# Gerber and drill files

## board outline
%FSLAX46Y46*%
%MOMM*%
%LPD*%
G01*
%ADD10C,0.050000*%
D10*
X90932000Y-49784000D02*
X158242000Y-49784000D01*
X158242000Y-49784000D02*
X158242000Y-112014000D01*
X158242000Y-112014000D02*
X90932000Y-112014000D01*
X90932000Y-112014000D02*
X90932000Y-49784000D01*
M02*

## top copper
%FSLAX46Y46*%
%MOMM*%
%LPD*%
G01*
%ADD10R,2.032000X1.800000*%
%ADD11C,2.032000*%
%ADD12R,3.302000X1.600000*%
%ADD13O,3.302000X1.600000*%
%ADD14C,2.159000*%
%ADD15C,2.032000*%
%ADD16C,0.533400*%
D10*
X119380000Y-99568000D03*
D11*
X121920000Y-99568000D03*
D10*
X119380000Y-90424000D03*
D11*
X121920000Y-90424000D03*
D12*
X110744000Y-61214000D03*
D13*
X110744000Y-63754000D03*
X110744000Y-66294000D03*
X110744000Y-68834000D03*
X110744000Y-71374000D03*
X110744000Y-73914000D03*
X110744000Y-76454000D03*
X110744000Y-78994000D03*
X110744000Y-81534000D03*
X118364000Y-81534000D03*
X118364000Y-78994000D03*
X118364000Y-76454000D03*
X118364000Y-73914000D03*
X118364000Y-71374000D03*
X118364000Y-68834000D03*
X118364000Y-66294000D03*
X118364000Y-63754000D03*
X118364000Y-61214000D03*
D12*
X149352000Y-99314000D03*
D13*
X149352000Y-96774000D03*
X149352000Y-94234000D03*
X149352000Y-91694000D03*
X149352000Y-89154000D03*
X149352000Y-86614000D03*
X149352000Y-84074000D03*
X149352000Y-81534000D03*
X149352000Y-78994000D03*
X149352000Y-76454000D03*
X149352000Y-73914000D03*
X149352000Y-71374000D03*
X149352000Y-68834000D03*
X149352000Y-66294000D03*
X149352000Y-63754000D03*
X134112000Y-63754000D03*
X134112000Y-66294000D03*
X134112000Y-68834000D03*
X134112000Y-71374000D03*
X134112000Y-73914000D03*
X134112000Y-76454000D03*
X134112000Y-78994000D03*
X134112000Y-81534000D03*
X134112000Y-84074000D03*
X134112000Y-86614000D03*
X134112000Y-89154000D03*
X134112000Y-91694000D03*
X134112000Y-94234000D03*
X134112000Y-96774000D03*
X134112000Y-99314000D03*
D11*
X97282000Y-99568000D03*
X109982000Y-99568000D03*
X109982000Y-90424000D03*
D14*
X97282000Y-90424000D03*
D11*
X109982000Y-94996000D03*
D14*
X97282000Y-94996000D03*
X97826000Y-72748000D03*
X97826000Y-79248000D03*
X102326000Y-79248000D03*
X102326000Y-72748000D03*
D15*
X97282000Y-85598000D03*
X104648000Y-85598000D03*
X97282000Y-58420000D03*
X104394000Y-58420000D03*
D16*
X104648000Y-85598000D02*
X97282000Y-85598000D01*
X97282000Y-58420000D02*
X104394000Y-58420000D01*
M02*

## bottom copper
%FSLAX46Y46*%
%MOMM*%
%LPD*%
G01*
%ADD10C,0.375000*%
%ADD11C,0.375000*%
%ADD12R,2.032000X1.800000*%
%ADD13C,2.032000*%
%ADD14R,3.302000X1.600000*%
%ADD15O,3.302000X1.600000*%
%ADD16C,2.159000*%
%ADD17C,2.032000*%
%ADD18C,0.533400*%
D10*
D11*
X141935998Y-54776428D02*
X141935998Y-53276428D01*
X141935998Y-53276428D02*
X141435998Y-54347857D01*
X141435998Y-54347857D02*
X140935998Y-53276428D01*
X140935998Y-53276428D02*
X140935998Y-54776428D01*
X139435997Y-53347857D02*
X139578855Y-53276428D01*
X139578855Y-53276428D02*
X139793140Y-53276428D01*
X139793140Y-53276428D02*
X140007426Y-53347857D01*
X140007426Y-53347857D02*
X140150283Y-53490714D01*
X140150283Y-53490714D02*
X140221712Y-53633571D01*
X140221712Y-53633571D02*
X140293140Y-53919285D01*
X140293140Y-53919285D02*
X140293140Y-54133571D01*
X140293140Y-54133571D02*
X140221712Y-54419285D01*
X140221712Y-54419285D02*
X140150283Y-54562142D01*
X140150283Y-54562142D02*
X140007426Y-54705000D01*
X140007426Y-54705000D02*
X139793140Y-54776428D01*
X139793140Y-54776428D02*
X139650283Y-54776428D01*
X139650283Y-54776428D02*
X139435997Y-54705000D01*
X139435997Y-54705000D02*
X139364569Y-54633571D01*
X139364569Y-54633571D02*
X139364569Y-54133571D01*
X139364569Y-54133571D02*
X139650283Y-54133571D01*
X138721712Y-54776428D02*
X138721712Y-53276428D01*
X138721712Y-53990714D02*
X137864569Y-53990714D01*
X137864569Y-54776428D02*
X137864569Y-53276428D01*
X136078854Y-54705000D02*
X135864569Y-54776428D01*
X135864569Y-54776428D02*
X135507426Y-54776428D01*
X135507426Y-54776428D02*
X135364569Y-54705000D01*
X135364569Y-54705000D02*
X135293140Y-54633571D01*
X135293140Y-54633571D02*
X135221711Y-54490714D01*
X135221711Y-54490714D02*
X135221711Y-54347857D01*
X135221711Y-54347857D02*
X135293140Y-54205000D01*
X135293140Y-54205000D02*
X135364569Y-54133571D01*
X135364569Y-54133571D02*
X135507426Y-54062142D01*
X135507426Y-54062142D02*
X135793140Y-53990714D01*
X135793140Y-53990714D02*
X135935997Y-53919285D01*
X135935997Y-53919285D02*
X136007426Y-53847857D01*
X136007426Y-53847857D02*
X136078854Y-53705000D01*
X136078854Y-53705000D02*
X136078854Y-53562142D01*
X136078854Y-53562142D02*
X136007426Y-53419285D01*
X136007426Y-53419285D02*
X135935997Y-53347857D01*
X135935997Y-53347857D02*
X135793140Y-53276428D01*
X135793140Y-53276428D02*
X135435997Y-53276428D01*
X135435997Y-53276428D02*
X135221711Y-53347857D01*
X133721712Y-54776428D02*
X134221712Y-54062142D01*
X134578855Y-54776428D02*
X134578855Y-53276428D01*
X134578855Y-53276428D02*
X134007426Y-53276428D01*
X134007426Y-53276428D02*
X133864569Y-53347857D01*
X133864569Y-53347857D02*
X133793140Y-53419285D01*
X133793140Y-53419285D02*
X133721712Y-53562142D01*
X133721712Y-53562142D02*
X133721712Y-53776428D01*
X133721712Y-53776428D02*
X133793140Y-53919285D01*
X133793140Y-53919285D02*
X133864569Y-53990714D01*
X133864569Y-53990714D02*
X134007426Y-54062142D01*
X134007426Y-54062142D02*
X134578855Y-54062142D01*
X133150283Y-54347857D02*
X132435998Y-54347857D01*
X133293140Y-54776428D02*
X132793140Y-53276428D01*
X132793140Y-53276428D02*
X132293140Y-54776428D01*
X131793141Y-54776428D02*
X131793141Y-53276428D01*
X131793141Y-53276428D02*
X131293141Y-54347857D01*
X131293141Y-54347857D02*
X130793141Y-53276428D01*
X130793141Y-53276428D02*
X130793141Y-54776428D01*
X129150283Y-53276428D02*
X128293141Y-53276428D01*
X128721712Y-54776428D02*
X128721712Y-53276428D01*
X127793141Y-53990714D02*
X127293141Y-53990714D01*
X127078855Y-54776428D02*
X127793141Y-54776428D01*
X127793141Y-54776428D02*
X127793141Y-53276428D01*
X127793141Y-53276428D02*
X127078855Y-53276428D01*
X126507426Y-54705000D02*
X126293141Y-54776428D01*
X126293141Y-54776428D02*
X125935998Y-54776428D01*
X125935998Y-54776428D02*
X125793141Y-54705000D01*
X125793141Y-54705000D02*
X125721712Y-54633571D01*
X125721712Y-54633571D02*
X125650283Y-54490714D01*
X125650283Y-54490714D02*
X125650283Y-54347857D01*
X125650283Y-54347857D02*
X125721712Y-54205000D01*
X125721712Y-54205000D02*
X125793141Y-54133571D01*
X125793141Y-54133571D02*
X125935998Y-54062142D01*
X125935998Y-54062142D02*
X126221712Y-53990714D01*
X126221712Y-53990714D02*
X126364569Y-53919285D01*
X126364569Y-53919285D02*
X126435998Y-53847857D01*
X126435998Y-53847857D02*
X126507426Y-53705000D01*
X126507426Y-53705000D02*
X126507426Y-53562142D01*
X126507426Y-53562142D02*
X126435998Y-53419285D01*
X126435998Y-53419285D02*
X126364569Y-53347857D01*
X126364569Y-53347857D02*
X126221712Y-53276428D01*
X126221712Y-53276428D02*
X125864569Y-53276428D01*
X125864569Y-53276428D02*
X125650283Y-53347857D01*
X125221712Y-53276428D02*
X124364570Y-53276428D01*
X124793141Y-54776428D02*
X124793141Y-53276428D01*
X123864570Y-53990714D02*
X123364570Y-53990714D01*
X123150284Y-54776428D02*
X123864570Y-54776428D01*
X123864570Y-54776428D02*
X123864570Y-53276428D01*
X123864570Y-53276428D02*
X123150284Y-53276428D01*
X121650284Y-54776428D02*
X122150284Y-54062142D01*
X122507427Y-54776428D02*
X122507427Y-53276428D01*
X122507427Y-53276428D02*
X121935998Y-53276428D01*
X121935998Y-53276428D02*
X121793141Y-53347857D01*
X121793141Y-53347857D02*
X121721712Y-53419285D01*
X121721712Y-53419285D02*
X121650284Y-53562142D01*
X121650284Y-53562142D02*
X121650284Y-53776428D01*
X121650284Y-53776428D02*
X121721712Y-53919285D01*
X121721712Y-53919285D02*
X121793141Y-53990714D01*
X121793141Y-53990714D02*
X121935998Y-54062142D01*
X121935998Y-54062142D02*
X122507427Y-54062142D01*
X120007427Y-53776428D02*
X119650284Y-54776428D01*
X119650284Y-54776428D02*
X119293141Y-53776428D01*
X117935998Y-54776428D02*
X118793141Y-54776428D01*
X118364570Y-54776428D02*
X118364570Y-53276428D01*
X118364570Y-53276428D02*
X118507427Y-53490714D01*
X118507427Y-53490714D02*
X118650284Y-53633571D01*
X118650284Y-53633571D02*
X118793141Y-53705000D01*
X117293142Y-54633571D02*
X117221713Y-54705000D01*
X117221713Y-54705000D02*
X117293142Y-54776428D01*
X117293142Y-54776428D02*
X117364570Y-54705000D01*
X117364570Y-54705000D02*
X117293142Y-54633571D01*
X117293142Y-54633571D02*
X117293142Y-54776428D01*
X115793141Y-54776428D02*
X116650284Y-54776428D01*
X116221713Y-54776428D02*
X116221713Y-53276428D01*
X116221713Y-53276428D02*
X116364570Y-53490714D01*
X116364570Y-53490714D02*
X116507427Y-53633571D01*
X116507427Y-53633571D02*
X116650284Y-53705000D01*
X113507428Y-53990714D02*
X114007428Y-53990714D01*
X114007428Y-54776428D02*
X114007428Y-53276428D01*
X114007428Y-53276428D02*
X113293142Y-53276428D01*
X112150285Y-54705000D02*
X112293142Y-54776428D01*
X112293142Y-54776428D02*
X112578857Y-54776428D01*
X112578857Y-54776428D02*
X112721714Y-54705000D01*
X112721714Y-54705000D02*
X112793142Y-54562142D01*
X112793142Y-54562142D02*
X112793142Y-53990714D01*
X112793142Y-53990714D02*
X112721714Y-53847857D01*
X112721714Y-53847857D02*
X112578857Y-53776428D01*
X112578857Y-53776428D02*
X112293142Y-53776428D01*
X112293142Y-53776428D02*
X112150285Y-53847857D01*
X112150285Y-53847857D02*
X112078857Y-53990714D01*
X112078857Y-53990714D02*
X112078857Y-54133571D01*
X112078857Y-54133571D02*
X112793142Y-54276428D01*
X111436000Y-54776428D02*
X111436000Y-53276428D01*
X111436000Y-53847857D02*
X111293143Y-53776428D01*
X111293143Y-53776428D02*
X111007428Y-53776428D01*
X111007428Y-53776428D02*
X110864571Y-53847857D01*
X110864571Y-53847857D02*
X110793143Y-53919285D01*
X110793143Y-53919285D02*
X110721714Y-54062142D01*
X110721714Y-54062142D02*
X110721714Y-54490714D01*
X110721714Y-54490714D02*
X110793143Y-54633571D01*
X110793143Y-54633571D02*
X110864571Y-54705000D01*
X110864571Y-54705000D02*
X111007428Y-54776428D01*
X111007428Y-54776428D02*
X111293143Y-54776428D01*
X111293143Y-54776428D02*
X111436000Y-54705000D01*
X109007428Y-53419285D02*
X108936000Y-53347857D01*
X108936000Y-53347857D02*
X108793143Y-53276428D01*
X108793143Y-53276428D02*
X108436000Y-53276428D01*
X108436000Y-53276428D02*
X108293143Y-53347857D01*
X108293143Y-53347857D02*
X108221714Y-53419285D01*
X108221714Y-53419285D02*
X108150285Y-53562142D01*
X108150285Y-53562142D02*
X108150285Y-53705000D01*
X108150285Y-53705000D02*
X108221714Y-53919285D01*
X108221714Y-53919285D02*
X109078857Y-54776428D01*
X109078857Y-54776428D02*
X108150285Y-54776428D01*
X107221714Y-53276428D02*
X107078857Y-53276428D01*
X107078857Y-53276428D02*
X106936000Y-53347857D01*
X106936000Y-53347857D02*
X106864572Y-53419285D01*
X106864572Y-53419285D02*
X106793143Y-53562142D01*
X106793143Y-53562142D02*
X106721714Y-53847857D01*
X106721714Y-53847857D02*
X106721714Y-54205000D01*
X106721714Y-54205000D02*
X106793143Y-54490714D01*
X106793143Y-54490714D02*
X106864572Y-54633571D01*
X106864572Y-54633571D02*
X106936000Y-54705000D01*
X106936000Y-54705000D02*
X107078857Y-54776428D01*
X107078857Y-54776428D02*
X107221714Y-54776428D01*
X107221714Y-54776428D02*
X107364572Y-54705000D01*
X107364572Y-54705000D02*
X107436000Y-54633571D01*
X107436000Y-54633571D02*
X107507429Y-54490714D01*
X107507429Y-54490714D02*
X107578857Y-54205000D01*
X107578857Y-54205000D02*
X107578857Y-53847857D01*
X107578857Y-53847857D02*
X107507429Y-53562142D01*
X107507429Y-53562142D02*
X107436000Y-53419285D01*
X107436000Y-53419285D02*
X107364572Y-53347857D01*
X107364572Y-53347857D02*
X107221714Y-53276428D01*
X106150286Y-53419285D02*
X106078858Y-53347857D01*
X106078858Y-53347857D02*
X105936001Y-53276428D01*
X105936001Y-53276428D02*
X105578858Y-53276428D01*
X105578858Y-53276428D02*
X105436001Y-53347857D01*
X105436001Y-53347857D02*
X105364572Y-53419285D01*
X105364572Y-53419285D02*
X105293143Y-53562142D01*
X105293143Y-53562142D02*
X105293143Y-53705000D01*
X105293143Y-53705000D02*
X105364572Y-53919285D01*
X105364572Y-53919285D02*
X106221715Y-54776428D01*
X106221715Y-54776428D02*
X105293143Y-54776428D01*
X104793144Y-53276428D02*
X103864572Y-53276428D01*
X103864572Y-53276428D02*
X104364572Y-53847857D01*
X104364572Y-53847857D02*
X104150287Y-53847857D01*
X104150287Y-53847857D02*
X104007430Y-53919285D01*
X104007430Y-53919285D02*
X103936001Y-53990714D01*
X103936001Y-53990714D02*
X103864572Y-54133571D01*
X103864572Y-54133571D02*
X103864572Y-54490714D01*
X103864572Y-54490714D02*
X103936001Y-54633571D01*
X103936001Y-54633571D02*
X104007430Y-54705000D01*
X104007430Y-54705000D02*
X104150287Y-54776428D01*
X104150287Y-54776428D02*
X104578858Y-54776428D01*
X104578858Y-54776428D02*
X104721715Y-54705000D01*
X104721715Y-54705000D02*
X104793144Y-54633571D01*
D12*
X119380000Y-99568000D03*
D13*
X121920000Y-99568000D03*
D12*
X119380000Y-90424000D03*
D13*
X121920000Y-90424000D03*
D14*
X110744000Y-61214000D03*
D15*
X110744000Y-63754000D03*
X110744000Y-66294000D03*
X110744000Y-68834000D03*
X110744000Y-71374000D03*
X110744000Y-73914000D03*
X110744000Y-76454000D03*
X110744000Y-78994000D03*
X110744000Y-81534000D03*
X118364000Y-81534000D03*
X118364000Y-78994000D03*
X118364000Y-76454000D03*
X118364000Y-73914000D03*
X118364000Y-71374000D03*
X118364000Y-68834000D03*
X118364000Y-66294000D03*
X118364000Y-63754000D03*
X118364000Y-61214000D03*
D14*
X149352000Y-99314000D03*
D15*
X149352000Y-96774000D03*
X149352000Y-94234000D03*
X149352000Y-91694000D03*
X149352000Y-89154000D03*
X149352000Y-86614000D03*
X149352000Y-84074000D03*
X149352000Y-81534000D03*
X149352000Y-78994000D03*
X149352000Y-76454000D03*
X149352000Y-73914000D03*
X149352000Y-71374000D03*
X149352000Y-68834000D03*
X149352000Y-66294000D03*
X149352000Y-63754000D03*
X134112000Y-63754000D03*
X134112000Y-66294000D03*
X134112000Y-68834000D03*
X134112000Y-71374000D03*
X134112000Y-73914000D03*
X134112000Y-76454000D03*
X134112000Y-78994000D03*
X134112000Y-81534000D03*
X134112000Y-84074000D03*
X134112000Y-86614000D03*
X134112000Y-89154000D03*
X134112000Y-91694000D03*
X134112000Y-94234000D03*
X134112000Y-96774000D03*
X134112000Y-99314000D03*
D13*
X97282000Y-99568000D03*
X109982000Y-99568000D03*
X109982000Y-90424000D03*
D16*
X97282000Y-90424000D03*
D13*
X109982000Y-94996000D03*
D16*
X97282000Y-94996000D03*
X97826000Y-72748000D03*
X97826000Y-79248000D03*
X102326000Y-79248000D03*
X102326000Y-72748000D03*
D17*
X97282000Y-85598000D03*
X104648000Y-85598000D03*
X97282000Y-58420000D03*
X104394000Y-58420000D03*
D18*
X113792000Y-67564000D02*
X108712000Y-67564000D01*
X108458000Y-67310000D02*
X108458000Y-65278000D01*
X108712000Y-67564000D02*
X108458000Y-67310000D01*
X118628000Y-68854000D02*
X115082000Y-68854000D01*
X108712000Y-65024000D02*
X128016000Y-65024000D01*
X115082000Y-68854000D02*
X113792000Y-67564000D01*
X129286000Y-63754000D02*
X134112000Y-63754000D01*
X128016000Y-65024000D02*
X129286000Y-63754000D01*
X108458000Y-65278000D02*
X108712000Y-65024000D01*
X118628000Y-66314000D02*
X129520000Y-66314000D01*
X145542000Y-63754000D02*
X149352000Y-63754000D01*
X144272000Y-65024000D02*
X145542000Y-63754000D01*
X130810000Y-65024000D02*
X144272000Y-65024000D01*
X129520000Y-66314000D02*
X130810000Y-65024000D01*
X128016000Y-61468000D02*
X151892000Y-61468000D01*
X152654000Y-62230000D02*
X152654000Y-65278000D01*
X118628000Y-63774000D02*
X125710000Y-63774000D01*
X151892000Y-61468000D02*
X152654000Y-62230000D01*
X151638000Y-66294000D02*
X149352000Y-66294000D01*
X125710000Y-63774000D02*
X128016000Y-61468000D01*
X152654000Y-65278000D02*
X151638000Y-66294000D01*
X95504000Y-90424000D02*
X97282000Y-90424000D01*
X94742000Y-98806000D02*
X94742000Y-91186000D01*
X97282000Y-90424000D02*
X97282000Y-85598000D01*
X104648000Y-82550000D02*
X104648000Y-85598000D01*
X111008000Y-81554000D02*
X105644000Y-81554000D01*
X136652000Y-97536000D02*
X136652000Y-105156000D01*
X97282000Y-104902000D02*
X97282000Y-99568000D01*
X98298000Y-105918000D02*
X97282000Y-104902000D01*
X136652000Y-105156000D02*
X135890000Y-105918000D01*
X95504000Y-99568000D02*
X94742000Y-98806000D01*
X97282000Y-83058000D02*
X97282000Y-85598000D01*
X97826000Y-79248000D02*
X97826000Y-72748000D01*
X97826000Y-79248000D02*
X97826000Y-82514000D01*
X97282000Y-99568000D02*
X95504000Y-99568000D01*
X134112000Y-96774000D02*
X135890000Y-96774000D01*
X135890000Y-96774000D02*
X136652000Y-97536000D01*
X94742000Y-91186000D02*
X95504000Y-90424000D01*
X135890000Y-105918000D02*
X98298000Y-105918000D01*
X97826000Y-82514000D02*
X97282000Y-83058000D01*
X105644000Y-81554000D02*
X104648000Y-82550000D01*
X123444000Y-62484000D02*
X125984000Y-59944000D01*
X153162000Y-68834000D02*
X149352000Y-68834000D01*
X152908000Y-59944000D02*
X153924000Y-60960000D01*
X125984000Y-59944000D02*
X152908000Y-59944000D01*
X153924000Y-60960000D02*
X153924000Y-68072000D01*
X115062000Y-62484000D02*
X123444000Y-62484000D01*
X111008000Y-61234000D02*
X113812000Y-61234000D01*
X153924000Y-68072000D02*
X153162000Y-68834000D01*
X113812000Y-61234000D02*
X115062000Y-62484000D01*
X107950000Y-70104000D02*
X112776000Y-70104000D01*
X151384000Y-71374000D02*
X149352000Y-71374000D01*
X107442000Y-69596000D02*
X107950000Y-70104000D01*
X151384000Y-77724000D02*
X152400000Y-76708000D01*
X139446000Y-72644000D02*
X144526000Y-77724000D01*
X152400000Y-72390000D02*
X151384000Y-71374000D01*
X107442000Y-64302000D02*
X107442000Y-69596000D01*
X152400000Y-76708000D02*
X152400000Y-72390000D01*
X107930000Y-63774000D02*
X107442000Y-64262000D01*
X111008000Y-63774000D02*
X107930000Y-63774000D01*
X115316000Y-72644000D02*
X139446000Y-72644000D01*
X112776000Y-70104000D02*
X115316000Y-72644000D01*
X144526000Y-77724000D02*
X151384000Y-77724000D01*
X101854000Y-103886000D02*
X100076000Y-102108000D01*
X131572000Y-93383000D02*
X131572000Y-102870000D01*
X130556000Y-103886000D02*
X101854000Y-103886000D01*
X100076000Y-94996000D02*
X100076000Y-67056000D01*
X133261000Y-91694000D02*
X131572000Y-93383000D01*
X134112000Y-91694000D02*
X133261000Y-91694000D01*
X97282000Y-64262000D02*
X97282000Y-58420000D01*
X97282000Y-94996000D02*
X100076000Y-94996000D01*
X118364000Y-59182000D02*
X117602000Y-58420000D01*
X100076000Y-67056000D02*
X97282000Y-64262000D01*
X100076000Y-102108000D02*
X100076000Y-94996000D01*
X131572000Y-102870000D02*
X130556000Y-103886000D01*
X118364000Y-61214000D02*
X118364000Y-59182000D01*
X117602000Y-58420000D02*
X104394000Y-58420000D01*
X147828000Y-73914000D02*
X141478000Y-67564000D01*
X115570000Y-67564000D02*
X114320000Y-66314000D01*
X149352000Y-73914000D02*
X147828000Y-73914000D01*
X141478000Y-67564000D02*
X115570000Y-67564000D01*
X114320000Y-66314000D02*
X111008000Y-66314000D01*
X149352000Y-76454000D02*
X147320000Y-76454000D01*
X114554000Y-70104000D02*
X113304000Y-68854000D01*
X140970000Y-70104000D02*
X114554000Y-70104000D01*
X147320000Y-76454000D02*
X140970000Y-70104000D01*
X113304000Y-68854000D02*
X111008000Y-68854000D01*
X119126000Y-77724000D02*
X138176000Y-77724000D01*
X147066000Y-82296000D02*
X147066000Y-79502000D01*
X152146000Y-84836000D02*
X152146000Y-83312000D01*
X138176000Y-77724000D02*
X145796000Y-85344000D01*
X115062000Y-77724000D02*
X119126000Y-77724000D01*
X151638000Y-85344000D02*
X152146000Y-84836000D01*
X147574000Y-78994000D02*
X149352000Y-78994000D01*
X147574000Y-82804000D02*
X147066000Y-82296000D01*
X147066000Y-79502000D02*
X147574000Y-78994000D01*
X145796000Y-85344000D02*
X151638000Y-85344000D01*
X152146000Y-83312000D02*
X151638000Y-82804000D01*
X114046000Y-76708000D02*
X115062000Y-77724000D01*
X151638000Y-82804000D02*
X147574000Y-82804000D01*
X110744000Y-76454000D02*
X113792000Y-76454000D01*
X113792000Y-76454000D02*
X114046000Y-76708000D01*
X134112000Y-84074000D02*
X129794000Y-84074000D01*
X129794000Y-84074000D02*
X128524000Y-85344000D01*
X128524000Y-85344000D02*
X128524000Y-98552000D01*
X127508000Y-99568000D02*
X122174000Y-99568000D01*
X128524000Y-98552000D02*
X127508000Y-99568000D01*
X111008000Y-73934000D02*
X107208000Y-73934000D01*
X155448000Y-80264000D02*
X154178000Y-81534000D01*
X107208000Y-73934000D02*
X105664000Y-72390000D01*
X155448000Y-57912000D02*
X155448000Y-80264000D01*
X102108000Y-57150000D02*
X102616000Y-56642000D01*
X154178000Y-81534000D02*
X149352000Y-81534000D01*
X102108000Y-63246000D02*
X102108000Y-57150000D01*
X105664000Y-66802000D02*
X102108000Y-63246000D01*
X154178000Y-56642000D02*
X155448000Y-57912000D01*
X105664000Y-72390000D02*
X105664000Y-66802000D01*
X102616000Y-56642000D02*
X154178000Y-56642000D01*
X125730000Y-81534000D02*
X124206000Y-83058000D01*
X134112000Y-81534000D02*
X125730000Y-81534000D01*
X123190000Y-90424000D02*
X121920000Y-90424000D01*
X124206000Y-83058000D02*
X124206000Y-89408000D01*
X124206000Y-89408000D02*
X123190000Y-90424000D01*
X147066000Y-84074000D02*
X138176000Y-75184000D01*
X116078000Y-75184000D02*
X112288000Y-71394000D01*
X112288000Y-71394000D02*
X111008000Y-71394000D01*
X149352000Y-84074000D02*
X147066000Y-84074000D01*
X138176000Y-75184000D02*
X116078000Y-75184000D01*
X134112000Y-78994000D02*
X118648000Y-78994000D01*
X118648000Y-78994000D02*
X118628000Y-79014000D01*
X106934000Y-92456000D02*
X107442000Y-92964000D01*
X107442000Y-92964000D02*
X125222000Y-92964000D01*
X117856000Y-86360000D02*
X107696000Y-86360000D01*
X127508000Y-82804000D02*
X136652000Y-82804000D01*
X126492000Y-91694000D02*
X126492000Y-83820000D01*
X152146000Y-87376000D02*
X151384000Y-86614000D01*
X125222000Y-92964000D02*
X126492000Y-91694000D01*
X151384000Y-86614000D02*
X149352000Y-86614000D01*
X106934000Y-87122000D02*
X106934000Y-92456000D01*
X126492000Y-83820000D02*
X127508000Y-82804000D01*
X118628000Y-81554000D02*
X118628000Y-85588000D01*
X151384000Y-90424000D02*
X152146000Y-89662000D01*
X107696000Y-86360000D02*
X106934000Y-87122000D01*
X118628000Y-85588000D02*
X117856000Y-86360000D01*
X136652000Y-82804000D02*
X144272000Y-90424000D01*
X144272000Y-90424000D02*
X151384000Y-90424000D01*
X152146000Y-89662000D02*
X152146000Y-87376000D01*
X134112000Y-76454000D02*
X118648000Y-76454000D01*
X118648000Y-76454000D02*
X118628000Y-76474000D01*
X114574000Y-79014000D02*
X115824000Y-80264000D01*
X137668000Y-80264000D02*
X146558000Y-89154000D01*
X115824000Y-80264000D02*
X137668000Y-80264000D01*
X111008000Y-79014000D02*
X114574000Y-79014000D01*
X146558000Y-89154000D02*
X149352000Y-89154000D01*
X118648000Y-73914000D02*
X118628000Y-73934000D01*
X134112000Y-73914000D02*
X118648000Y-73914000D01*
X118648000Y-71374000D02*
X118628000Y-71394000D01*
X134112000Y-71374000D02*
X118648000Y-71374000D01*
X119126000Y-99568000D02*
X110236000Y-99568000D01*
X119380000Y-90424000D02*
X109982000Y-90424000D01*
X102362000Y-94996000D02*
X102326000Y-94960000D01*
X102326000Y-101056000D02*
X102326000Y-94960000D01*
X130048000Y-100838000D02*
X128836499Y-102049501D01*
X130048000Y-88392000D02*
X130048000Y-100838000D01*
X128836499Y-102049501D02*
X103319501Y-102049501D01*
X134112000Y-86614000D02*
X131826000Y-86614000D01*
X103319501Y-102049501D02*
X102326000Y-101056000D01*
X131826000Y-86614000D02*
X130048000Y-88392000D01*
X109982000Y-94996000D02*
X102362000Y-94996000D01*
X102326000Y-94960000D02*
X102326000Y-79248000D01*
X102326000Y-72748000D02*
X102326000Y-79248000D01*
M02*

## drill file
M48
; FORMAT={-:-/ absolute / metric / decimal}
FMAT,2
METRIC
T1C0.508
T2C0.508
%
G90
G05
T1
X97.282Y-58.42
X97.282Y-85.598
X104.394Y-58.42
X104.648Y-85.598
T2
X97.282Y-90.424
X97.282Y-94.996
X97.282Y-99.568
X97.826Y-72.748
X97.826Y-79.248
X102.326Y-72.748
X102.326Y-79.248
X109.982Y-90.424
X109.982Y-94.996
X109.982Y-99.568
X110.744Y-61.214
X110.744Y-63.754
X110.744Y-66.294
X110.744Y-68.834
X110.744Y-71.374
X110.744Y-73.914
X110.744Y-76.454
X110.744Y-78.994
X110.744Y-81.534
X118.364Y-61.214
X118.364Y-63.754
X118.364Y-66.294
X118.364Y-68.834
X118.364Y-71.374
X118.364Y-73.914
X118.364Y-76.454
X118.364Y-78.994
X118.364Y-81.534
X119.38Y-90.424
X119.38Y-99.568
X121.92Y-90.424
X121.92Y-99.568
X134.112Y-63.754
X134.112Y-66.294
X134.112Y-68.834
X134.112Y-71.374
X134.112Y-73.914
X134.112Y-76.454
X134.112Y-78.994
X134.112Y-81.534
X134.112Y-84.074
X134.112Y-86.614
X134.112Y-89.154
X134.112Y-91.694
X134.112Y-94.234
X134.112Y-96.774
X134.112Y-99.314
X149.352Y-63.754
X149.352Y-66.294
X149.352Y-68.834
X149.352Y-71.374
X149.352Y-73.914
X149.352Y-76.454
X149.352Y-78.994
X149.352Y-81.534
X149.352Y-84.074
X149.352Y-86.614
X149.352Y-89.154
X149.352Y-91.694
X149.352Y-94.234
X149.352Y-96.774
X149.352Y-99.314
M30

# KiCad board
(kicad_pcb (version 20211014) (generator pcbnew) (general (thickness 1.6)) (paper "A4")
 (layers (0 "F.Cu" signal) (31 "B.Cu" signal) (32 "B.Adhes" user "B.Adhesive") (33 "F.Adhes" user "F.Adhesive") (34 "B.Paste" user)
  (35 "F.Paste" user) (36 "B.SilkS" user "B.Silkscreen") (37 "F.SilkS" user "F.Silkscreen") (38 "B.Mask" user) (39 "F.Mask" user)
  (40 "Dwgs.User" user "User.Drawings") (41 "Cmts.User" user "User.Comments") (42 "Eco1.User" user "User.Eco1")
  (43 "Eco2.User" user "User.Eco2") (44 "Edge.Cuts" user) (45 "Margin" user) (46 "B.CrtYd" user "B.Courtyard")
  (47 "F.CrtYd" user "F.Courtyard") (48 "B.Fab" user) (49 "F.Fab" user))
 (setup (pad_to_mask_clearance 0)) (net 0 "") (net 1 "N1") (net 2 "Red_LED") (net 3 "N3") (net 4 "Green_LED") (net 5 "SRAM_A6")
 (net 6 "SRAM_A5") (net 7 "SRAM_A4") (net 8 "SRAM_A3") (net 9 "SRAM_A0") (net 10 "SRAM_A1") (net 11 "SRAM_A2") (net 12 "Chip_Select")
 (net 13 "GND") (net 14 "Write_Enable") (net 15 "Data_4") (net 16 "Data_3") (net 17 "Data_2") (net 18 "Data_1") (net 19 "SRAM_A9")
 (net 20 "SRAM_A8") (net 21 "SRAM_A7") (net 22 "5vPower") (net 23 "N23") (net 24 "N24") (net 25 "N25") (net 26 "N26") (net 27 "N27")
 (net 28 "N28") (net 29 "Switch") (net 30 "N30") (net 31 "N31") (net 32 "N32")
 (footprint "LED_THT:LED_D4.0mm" (layer "F.Cu") (at 119.38 99.568)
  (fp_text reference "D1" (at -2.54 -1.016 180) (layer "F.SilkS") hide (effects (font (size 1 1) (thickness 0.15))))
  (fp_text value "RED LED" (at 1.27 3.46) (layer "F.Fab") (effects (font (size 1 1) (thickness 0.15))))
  (pad "1" thru_hole rect locked (at 0 0) (size 2.032 1.8) (drill 0.508) (layers *.Cu *.Mask) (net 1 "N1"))
  (pad "2" thru_hole circle locked (at 2.54 0) (size 2.032 2.032) (drill 0.508) (layers *.Cu *.Mask) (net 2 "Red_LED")))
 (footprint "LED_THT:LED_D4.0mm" (layer "F.Cu") (at 119.38 90.424)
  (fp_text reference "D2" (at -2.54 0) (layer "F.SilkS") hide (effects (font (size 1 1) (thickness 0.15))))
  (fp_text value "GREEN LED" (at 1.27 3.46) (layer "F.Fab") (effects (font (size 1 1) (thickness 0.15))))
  (pad "1" thru_hole rect locked (at 0 0) (size 2.032 1.8) (drill 0.508) (layers *.Cu *.Mask) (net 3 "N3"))
  (pad "2" thru_hole circle locked (at 2.54 0) (size 2.032 2.032) (drill 0.508) (layers *.Cu *.Mask) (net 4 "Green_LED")))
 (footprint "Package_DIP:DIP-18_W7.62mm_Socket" (layer "F.Cu") (at 110.744 61.214)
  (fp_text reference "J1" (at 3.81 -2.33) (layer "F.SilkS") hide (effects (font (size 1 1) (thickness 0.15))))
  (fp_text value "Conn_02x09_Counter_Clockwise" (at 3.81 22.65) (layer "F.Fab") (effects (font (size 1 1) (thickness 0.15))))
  (pad "1" thru_hole rect (at 0 0) (size 3.302 1.6) (drill 0.508) (layers *.Cu *.Mask) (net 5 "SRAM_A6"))
  (pad "2" thru_hole oval (at 0 2.54) (size 3.302 1.6) (drill 0.508) (layers *.Cu *.Mask) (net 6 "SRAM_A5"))
  (pad "3" thru_hole oval (at 0 5.08) (size 3.302 1.6) (drill 0.508) (layers *.Cu *.Mask) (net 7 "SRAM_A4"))
  (pad "4" thru_hole oval (at 0 7.62) (size 3.302 1.6) (drill 0.508) (layers *.Cu *.Mask) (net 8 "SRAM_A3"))
  (pad "5" thru_hole oval (at 0 10.16) (size 3.302 1.6) (drill 0.508) (layers *.Cu *.Mask) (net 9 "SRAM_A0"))
  (pad "6" thru_hole oval (at 0 12.7) (size 3.302 1.6) (drill 0.508) (layers *.Cu *.Mask) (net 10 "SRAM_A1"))
  (pad "7" thru_hole oval (at 0 15.24) (size 3.302 1.6) (drill 0.508) (layers *.Cu *.Mask) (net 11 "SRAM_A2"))
  (pad "8" thru_hole oval (at 0 17.78) (size 3.302 1.6) (drill 0.508) (layers *.Cu *.Mask) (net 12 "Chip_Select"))
  (pad "9" thru_hole oval (at 0 20.32) (size 3.302 1.6) (drill 0.508) (layers *.Cu *.Mask) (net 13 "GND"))
  (pad "10" thru_hole oval (at 7.62 20.32) (size 3.302 1.6) (drill 0.508) (layers *.Cu *.Mask) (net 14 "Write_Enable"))
  (pad "11" thru_hole oval (at 7.62 17.78) (size 3.302 1.6) (drill 0.508) (layers *.Cu *.Mask) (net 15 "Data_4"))
  (pad "12" thru_hole oval (at 7.62 15.24) (size 3.302 1.6) (drill 0.508) (layers *.Cu *.Mask) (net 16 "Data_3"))
  (pad "13" thru_hole oval (at 7.62 12.7) (size 3.302 1.6) (drill 0.508) (layers *.Cu *.Mask) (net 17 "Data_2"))
  (pad "14" thru_hole oval (at 7.62 10.16) (size 3.302 1.6) (drill 0.508) (layers *.Cu *.Mask) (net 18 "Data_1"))
  (pad "15" thru_hole oval (at 7.62 7.62) (size 3.302 1.6) (drill 0.508) (layers *.Cu *.Mask) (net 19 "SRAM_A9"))
  (pad "16" thru_hole oval (at 7.62 5.08) (size 3.302 1.6) (drill 0.508) (layers *.Cu *.Mask) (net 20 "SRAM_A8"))
  (pad "17" thru_hole oval (at 7.62 2.54) (size 3.302 1.6) (drill 0.508) (layers *.Cu *.Mask) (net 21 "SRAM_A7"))
  (pad "18" thru_hole oval (at 7.62 0) (size 3.302 1.6) (drill 0.508) (layers *.Cu *.Mask) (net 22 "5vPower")))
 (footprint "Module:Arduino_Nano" (layer "F.Cu") (at 149.352 99.314 180)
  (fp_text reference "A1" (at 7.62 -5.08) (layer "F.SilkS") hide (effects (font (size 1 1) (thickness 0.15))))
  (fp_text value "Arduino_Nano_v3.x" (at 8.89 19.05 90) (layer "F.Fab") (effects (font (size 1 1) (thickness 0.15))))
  (pad "1" thru_hole rect (at 0 0 180) (size 3.302 1.6) (drill 0.508) (layers *.Cu *.Mask) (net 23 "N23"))
  (pad "2" thru_hole oval (at 0 2.54 180) (size 3.302 1.6) (drill 0.508) (layers *.Cu *.Mask) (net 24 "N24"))
  (pad "3" thru_hole oval (at 0 5.08 180) (size 3.302 1.6) (drill 0.508) (layers *.Cu *.Mask) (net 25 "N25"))
  (pad "4" thru_hole oval (at 0 7.62 180) (size 3.302 1.6) (drill 0.508) (layers *.Cu *.Mask) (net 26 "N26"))
  (pad "5" thru_hole oval (at 0 10.16 180) (size 3.302 1.6) (drill 0.508) (layers *.Cu *.Mask) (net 12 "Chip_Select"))
  (pad "6" thru_hole oval (at 0 12.7 180) (size 3.302 1.6) (drill 0.508) (layers *.Cu *.Mask) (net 14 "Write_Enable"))
  (pad "7" thru_hole oval (at 0 15.24 180) (size 3.302 1.6) (drill 0.508) (layers *.Cu *.Mask) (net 9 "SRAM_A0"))
  (pad "8" thru_hole oval (at 0 17.78 180) (size 3.302 1.6) (drill 0.508) (layers *.Cu *.Mask) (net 10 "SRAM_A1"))
  (pad "9" thru_hole oval (at 0 20.32 180) (size 3.302 1.6) (drill 0.508) (layers *.Cu *.Mask) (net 11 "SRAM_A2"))
  (pad "10" thru_hole oval (at 0 22.86 180) (size 3.302 1.6) (drill 0.508) (layers *.Cu *.Mask) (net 8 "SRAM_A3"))
  (pad "11" thru_hole oval (at 0 25.4 180) (size 3.302 1.6) (drill 0.508) (layers *.Cu *.Mask) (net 7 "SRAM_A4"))
  (pad "12" thru_hole oval (at 0 27.94 180) (size 3.302 1.6) (drill 0.508) (layers *.Cu *.Mask) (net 6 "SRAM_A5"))
  (pad "13" thru_hole oval (at 0 30.48 180) (size 3.302 1.6) (drill 0.508) (layers *.Cu *.Mask) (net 5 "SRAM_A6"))
  (pad "14" thru_hole oval (at 0 33.02 180) (size 3.302 1.6) (drill 0.508) (layers *.Cu *.Mask) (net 21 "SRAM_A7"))
  (pad "15" thru_hole oval (at 0 35.56 180) (size 3.302 1.6) (drill 0.508) (layers *.Cu *.Mask) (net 20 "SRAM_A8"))
  (pad "16" thru_hole oval (at 15.24 35.56 180) (size 3.302 1.6) (drill 0.508) (layers *.Cu *.Mask) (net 19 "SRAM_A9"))
  (pad "17" thru_hole oval (at 15.24 33.02 180) (size 3.302 1.6) (drill 0.508) (layers *.Cu *.Mask) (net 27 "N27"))
  (pad "18" thru_hole oval (at 15.24 30.48 180) (size 3.302 1.6) (drill 0.508) (layers *.Cu *.Mask) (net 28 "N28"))
  (pad "19" thru_hole oval (at 15.24 27.94 180) (size 3.302 1.6) (drill 0.508) (layers *.Cu *.Mask) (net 18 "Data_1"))
  (pad "20" thru_hole oval (at 15.24 25.4 180) (size 3.302 1.6) (drill 0.508) (layers *.Cu *.Mask) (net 17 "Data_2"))
  (pad "21" thru_hole oval (at 15.24 22.86 180) (size 3.302 1.6) (drill 0.508) (layers *.Cu *.Mask) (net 16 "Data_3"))
  (pad "22" thru_hole oval (at 15.24 20.32 180) (size 3.302 1.6) (drill 0.508) (layers *.Cu *.Mask) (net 15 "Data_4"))
  (pad "23" thru_hole oval (at 15.24 17.78 180) (size 3.302 1.6) (drill 0.508) (layers *.Cu *.Mask) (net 4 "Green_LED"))
  (pad "24" thru_hole oval (at 15.24 15.24 180) (size 3.302 1.6) (drill 0.508) (layers *.Cu *.Mask) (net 2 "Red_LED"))
  (pad "25" thru_hole oval (at 15.24 12.7 180) (size 3.302 1.6) (drill 0.508) (layers *.Cu *.Mask) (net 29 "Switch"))
  (pad "26" thru_hole oval (at 15.24 10.16 180) (size 3.302 1.6) (drill 0.508) (layers *.Cu *.Mask) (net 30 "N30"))
  (pad "27" thru_hole oval (at 15.24 7.62 180) (size 3.302 1.6) (drill 0.508) (layers *.Cu *.Mask) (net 22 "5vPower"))
  (pad "28" thru_hole oval (at 15.24 5.08 180) (size 3.302 1.6) (drill 0.508) (layers *.Cu *.Mask) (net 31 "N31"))
  (pad "29" thru_hole oval (at 15.24 2.54 180) (size 3.302 1.6) (drill 0.508) (layers *.Cu *.Mask) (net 13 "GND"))
  (pad "30" thru_hole oval (at 15.24 0 180) (size 3.302 1.6) (drill 0.508) (layers *.Cu *.Mask) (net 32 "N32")))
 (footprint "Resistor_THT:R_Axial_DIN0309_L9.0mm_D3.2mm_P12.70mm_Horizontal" (layer "F.Cu") (at 97.282 99.568)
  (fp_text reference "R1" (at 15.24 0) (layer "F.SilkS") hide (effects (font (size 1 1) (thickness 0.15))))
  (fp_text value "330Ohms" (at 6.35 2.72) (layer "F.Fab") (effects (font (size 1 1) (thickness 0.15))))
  (pad "1" thru_hole circle locked (at 0 0) (size 2.032 2.032) (drill 0.508) (layers *.Cu *.Mask) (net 13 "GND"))
  (pad "2" thru_hole circle locked (at 12.7 0) (size 2.032 2.032) (drill 0.508) (layers *.Cu *.Mask) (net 1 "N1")))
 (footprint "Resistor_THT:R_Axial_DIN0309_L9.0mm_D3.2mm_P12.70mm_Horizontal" (layer "F.Cu") (at 109.982 90.424 180)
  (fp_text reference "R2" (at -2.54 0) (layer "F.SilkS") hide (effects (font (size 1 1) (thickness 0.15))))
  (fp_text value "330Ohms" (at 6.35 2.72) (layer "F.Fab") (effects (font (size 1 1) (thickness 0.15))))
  (pad "1" thru_hole circle locked (at 0 0 180) (size 2.032 2.032) (drill 0.508) (layers *.Cu *.Mask) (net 3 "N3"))
  (pad "2" thru_hole circle locked (at 12.7 0 180) (size 2.159 2.159) (drill 0.508) (layers *.Cu *.Mask) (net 13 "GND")))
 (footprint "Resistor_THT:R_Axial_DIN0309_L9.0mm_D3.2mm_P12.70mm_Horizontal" (layer "F.Cu") (at 109.982 94.996 180)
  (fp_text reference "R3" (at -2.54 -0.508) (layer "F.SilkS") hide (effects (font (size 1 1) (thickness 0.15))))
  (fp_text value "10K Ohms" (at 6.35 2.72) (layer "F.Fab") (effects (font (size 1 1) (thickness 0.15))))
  (pad "1" thru_hole circle locked (at 0 0 180) (size 2.032 2.032) (drill 0.508) (layers *.Cu *.Mask) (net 29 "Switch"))
  (pad "2" thru_hole circle locked (at 12.7 0 180) (size 2.159 2.159) (drill 0.508) (layers *.Cu *.Mask) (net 22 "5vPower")))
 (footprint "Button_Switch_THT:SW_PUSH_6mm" (layer "F.Cu") (at 97.826 79.248 90)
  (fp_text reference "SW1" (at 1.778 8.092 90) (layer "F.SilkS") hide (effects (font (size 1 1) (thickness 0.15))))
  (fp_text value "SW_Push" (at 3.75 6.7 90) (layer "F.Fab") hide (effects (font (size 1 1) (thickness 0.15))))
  (pad "1" thru_hole circle locked (at 6.5 0 180) (size 2.159 2.159) (drill 0.508) (layers *.Cu *.Mask) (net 13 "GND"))
  (pad "1" thru_hole circle locked (at 0 0 180) (size 2.159 2.159) (drill 0.508) (layers *.Cu *.Mask) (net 13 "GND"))
  (pad "2" thru_hole circle locked (at 0 4.5 180) (size 2.159 2.159) (drill 0.508) (layers *.Cu *.Mask) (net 29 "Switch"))
  (pad "2" thru_hole circle locked (at 6.5 4.5 180) (size 2.159 2.159) (drill 0.508) (layers *.Cu *.Mask) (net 29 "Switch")))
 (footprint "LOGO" (layer "F.Cu") (at 103.632 107.188)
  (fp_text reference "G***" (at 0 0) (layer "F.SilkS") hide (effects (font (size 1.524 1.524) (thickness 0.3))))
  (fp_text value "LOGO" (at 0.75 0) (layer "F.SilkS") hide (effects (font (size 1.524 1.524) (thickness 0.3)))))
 (gr_line (start 90.932 49.784) (end 158.242 49.784) (layer "Edge.Cuts") (width 0.05))
 (gr_line (start 158.242 49.784) (end 158.242 112.014) (layer "Edge.Cuts") (width 0.05))
 (gr_line (start 158.242 112.014) (end 90.932 112.014) (layer "Edge.Cuts") (width 0.05))
 (gr_line (start 90.932 112.014) (end 90.932 49.784) (layer "Edge.Cuts") (width 0.05))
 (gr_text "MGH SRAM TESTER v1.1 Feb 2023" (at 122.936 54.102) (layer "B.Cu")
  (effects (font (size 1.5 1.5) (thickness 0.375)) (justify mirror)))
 (segment (start 113.792 67.564) (end 108.712 67.564) (width 0.5334) (layer "B.Cu") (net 19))
 (segment (start 108.458 67.31) (end 108.458 65.278) (width 0.5334) (layer "B.Cu") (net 19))
 (segment (start 108.712 67.564) (end 108.458 67.31) (width 0.5334) (layer "B.Cu") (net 19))
 (segment (start 118.628 68.854) (end 115.082 68.854) (width 0.5334) (layer "B.Cu") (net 19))
 (segment (start 108.712 65.024) (end 128.016 65.024) (width 0.5334) (layer "B.Cu") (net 19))
 (segment (start 115.082 68.854) (end 113.792 67.564) (width 0.5334) (layer "B.Cu") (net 19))
 (segment (start 129.286 63.754) (end 134.112 63.754) (width 0.5334) (layer "B.Cu") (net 19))
 (segment (start 128.016 65.024) (end 129.286 63.754) (width 0.5334) (layer "B.Cu") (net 19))
 (segment (start 108.458 65.278) (end 108.712 65.024) (width 0.5334) (layer "B.Cu") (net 19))
 (segment (start 118.628 66.314) (end 129.52 66.314) (width 0.5334) (layer "B.Cu") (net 20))
 (segment (start 145.542 63.754) (end 149.352 63.754) (width 0.5334) (layer "B.Cu") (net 20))
 (segment (start 144.272 65.024) (end 145.542 63.754) (width 0.5334) (layer "B.Cu") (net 20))
 (segment (start 130.81 65.024) (end 144.272 65.024) (width 0.5334) (layer "B.Cu") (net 20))
 (segment (start 129.52 66.314) (end 130.81 65.024) (width 0.5334) (layer "B.Cu") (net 20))
 (segment (start 128.016 61.468) (end 151.892 61.468) (width 0.5334) (layer "B.Cu") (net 21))
 (segment (start 152.654 62.23) (end 152.654 65.278) (width 0.5334) (layer "B.Cu") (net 21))
 (segment (start 118.628 63.774) (end 125.71 63.774) (width 0.5334) (layer "B.Cu") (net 21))
 (segment (start 151.892 61.468) (end 152.654 62.23) (width 0.5334) (layer "B.Cu") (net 21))
 (segment (start 151.638 66.294) (end 149.352 66.294) (width 0.5334) (layer "B.Cu") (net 21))
 (segment (start 125.71 63.774) (end 128.016 61.468) (width 0.5334) (layer "B.Cu") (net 21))
 (segment (start 152.654 65.278) (end 151.638 66.294) (width 0.5334) (layer "B.Cu") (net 21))
 (segment (start 104.648 85.598) (end 97.282 85.598) (width 0.5334) (layer "F.Cu") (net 13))
 (via (at 97.282 85.598) (size 2.032) (drill 0.508) (layers "F.Cu" "B.Cu") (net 13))
 (via (at 104.648 85.598) (size 2.032) (drill 0.508) (layers "F.Cu" "B.Cu") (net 13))
 (segment (start 95.504 90.424) (end 97.282 90.424) (width 0.5334) (layer "B.Cu") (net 13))
 (segment (start 94.742 98.806) (end 94.742 91.186) (width 0.5334) (layer "B.Cu") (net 13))
 (segment (start 97.282 90.424) (end 97.282 85.598) (width 0.5334) (layer "B.Cu") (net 13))
 (segment (start 104.648 82.55) (end 104.648 85.598) (width 0.5334) (layer "B.Cu") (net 13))
 (segment (start 111.008 81.554) (end 105.644 81.554) (width 0.5334) (layer "B.Cu") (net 13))
 (segment (start 136.652 97.536) (end 136.652 105.156) (width 0.5334) (layer "B.Cu") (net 13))
 (segment (start 97.282 104.902) (end 97.282 99.568) (width 0.5334) (layer "B.Cu") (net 13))
 (segment (start 98.298 105.918) (end 97.282 104.902) (width 0.5334) (layer "B.Cu") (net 13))
 (segment (start 136.652 105.156) (end 135.89 105.918) (width 0.5334) (layer "B.Cu") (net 13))
 (segment (start 95.504 99.568) (end 94.742 98.806) (width 0.5334) (layer "B.Cu") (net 13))
 (segment (start 97.282 83.058) (end 97.282 85.598) (width 0.5334) (layer "B.Cu") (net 13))
 (segment (start 97.826 79.248) (end 97.826 72.748) (width 0.5334) (layer "B.Cu") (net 13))
 (segment (start 97.826 79.248) (end 97.826 82.514) (width 0.5334) (layer "B.Cu") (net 13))
 (segment (start 97.282 99.568) (end 95.504 99.568) (width 0.5334) (layer "B.Cu") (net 13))
 (segment (start 134.112 96.774) (end 135.89 96.774) (width 0.5334) (layer "B.Cu") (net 13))
 (segment (start 135.89 96.774) (end 136.652 97.536) (width 0.5334) (layer "B.Cu") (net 13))
 (segment (start 94.742 91.186) (end 95.504 90.424) (width 0.5334) (layer "B.Cu") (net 13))
 (segment (start 135.89 105.918) (end 98.298 105.918) (width 0.5334) (layer "B.Cu") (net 13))
 (segment (start 97.826 82.514) (end 97.282 83.058) (width 0.5334) (layer "B.Cu") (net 13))
 (segment (start 105.644 81.554) (end 104.648 82.55) (width 0.5334) (layer "B.Cu") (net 13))
 (segment (start 123.444 62.484) (end 125.984 59.944) (width 0.5334) (layer "B.Cu") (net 5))
 (segment (start 153.162 68.834) (end 149.352 68.834) (width 0.5334) (layer "B.Cu") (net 5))
 (segment (start 152.908 59.944) (end 153.924 60.96) (width 0.5334) (layer "B.Cu") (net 5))
 (segment (start 125.984 59.944) (end 152.908 59.944) (width 0.5334) (layer "B.Cu") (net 5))
 (segment (start 153.924 60.96) (end 153.924 68.072) (width 0.5334) (layer "B.Cu") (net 5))
 (segment (start 115.062 62.484) (end 123.444 62.484) (width 0.5334) (layer "B.Cu") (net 5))
 (segment (start 111.008 61.234) (end 113.812 61.234) (width 0.5334) (layer "B.Cu") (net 5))
 (segment (start 153.924 68.072) (end 153.162 68.834) (width 0.5334) (layer "B.Cu") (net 5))
 (segment (start 113.812 61.234) (end 115.062 62.484) (width 0.5334) (layer "B.Cu") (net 5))
 (segment (start 107.95 70.104) (end 112.776 70.104) (width 0.5334) (layer "B.Cu") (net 6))
 (segment (start 151.384 71.374) (end 149.352 71.374) (width 0.5334) (layer "B.Cu") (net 6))
 (segment (start 107.442 69.596) (end 107.95 70.104) (width 0.5334) (layer "B.Cu") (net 6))
 (segment (start 151.384 77.724) (end 152.4 76.708) (width 0.5334) (layer "B.Cu") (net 6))
 (segment (start 139.446 72.644) (end 144.526 77.724) (width 0.5334) (layer "B.Cu") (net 6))
 (segment (start 152.4 72.39) (end 151.384 71.374) (width 0.5334) (layer "B.Cu") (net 6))
 (segment (start 107.442 64.302) (end 107.442 69.596) (width 0.5334) (layer "B.Cu") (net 6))
 (segment (start 152.4 76.708) (end 152.4 72.39) (width 0.5334) (layer "B.Cu") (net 6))
 (segment (start 107.93 63.774) (end 107.442 64.262) (width 0.5334) (layer "B.Cu") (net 6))
 (segment (start 111.008 63.774) (end 107.93 63.774) (width 0.5334) (layer "B.Cu") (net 6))
 (segment (start 115.316 72.644) (end 139.446 72.644) (width 0.5334) (layer "B.Cu") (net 6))
 (segment (start 112.776 70.104) (end 115.316 72.644) (width 0.5334) (layer "B.Cu") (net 6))
 (segment (start 144.526 77.724) (end 151.384 77.724) (width 0.5334) (layer "B.Cu") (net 6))
 (segment (start 97.282 58.42) (end 104.394 58.42) (width 0.5334) (layer "F.Cu") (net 22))
 (via (at 97.282 58.42) (size 2.032) (drill 0.508) (layers "F.Cu" "B.Cu") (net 22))
 (via (at 104.394 58.42) (size 2.032) (drill 0.508) (layers "F.Cu" "B.Cu") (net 22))
 (segment (start 101.854 103.886) (end 100.076 102.108) (width 0.5334) (layer "B.Cu") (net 22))
 (segment (start 131.572 93.383) (end 131.572 102.87) (width 0.5334) (layer "B.Cu") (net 22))
 (segment (start 130.556 103.886) (end 101.854 103.886) (width 0.5334) (layer "B.Cu") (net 22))
 (segment (start 100.076 94.996) (end 100.076 67.056) (width 0.5334) (layer "B.Cu") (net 22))
 (segment (start 133.261 91.694) (end 131.572 93.383) (width 0.5334) (layer "B.Cu") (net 22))
 (segment (start 134.112 91.694) (end 133.261 91.694) (width 0.5334) (layer "B.Cu") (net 22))
 (segment (start 97.282 64.262) (end 97.282 58.42) (width 0.5334) (layer "B.Cu") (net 22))
 (segment (start 97.282 94.996) (end 100.076 94.996) (width 0.5334) (layer "B.Cu") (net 22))
 (segment (start 118.364 59.182) (end 117.602 58.42) (width 0.5334) (layer "B.Cu") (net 22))
 (segment (start 100.076 67.056) (end 97.282 64.262) (width 0.5334) (layer "B.Cu") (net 22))
 (segment (start 100.076 102.108) (end 100.076 94.996) (width 0.5334) (layer "B.Cu") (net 22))
 (segment (start 131.572 102.87) (end 130.556 103.886) (width 0.5334) (layer "B.Cu") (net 22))
 (segment (start 118.364 61.214) (end 118.364 59.182) (width 0.5334) (layer "B.Cu") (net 22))
 (segment (start 117.602 58.42) (end 104.394 58.42) (width 0.5334) (layer "B.Cu") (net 22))
 (segment (start 147.828 73.914) (end 141.478 67.564) (width 0.5334) (layer "B.Cu") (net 7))
 (segment (start 115.57 67.564) (end 114.32 66.314) (width 0.5334) (layer "B.Cu") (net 7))
 (segment (start 149.352 73.914) (end 147.828 73.914) (width 0.5334) (layer "B.Cu") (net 7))
 (segment (start 141.478 67.564) (end 115.57 67.564) (width 0.5334) (layer "B.Cu") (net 7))
 (segment (start 114.32 66.314) (end 111.008 66.314) (width 0.5334) (layer "B.Cu") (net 7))
 (segment (start 149.352 76.454) (end 147.32 76.454) (width 0.5334) (layer "B.Cu") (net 8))
 (segment (start 114.554 70.104) (end 113.304 68.854) (width 0.5334) (layer "B.Cu") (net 8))
 (segment (start 140.97 70.104) (end 114.554 70.104) (width 0.5334) (layer "B.Cu") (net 8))
 (segment (start 147.32 76.454) (end 140.97 70.104) (width 0.5334) (layer "B.Cu") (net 8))
 (segment (start 113.304 68.854) (end 111.008 68.854) (width 0.5334) (layer "B.Cu") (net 8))
 (segment (start 119.126 77.724) (end 138.176 77.724) (width 0.5334) (layer "B.Cu") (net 11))
 (segment (start 147.066 82.296) (end 147.066 79.502) (width 0.5334) (layer "B.Cu") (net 11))
 (segment (start 152.146 84.836) (end 152.146 83.312) (width 0.5334) (layer "B.Cu") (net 11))
 (segment (start 138.176 77.724) (end 145.796 85.344) (width 0.5334) (layer "B.Cu") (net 11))
 (segment (start 115.062 77.724) (end 119.126 77.724) (width 0.5334) (layer "B.Cu") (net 11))
 (segment (start 151.638 85.344) (end 152.146 84.836) (width 0.5334) (layer "B.Cu") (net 11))
 (segment (start 147.574 78.994) (end 149.352 78.994) (width 0.5334) (layer "B.Cu") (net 11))
 (segment (start 147.574 82.804) (end 147.066 82.296) (width 0.5334) (layer "B.Cu") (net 11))
 (segment (start 147.066 79.502) (end 147.574 78.994) (width 0.5334) (layer "B.Cu") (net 11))
 (segment (start 145.796 85.344) (end 151.638 85.344) (width 0.5334) (layer "B.Cu") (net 11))
 (segment (start 152.146 83.312) (end 151.638 82.804) (width 0.5334) (layer "B.Cu") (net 11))
 (segment (start 114.046 76.708) (end 115.062 77.724) (width 0.5334) (layer "B.Cu") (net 11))
 (segment (start 151.638 82.804) (end 147.574 82.804) (width 0.5334) (layer "B.Cu") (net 11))
 (segment (start 110.744 76.454) (end 113.792 76.454) (width 0.5334) (layer "B.Cu") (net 11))
 (segment (start 113.792 76.454) (end 114.046 76.708) (width 0.5334) (layer "B.Cu") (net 11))
 (segment (start 134.112 84.074) (end 129.794 84.074) (width 0.5334) (layer "B.Cu") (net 2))
 (segment (start 129.794 84.074) (end 128.524 85.344) (width 0.5334) (layer "B.Cu") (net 2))
 (segment (start 128.524 85.344) (end 128.524 98.552) (width 0.5334) (layer "B.Cu") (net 2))
 (segment (start 127.508 99.568) (end 122.174 99.568) (width 0.5334) (layer "B.Cu") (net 2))
 (segment (start 128.524 98.552) (end 127.508 99.568) (width 0.5334) (layer "B.Cu") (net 2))
 (segment (start 111.008 73.934) (end 107.208 73.934) (width 0.5334) (layer "B.Cu") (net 10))
 (segment (start 155.448 80.264) (end 154.178 81.534) (width 0.5334) (layer "B.Cu") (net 10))
 (segment (start 107.208 73.934) (end 105.664 72.39) (width 0.5334) (layer "B.Cu") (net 10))
 (segment (start 155.448 57.912) (end 155.448 80.264) (width 0.5334) (layer "B.Cu") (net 10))
 (segment (start 102.108 57.15) (end 102.616 56.642) (width 0.5334) (layer "B.Cu") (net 10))
 (segment (start 154.178 81.534) (end 149.352 81.534) (width 0.5334) (layer "B.Cu") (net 10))
 (segment (start 102.108 63.246) (end 102.108 57.15) (width 0.5334) (layer "B.Cu") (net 10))
 (segment (start 105.664 66.802) (end 102.108 63.246) (width 0.5334) (layer "B.Cu") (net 10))
 (segment (start 154.178 56.642) (end 155.448 57.912) (width 0.5334) (layer "B.Cu") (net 10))
 (segment (start 105.664 72.39) (end 105.664 66.802) (width 0.5334) (layer "B.Cu") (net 10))
 (segment (start 102.616 56.642) (end 154.178 56.642) (width 0.5334) (layer "B.Cu") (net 10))
 (segment (start 125.73 81.534) (end 124.206 83.058) (width 0.5334) (layer "B.Cu") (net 4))
 (segment (start 134.112 81.534) (end 125.73 81.534) (width 0.5334) (layer "B.Cu") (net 4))
 (segment (start 123.19 90.424) (end 121.92 90.424) (width 0.5334) (layer "B.Cu") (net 4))
 (segment (start 124.206 83.058) (end 124.206 89.408) (width 0.5334) (layer "B.Cu") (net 4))
 (segment (start 124.206 89.408) (end 123.19 90.424) (width 0.5334) (layer "B.Cu") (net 4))
 (segment (start 147.066 84.074) (end 138.176 75.184) (width 0.5334) (layer "B.Cu") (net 9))
 (segment (start 116.078 75.184) (end 112.288 71.394) (width 0.5334) (layer "B.Cu") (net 9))
 (segment (start 112.288 71.394) (end 111.008 71.394) (width 0.5334) (layer "B.Cu") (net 9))
 (segment (start 149.352 84.074) (end 147.066 84.074) (width 0.5334) (layer "B.Cu") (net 9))
 (segment (start 138.176 75.184) (end 116.078 75.184) (width 0.5334) (layer "B.Cu") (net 9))
 (segment (start 134.112 78.994) (end 118.648 78.994) (width 0.5334) (layer "B.Cu") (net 15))
 (segment (start 118.648 78.994) (end 118.628 79.014) (width 0.5334) (layer "B.Cu") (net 15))
 (segment (start 106.934 92.456) (end 107.442 92.964) (width 0.5334) (layer "B.Cu") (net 14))
 (segment (start 107.442 92.964) (end 125.222 92.964) (width 0.5334) (layer "B.Cu") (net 14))
 (segment (start 117.856 86.36) (end 107.696 86.36) (width 0.5334) (layer "B.Cu") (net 14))
 (segment (start 127.508 82.804) (end 136.652 82.804) (width 0.5334) (layer "B.Cu") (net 14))
 (segment (start 126.492 91.694) (end 126.492 83.82) (width 0.5334) (layer "B.Cu") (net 14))
 (segment (start 152.146 87.376) (end 151.384 86.614) (width 0.5334) (layer "B.Cu") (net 14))
 (segment (start 125.222 92.964) (end 126.492 91.694) (width 0.5334) (layer "B.Cu") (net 14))
 (segment (start 151.384 86.614) (end 149.352 86.614) (width 0.5334) (layer "B.Cu") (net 14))
 (segment (start 106.934 87.122) (end 106.934 92.456) (width 0.5334) (layer "B.Cu") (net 14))
 (segment (start 126.492 83.82) (end 127.508 82.804) (width 0.5334) (layer "B.Cu") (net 14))
 (segment (start 118.628 81.554) (end 118.628 85.588) (width 0.5334) (layer "B.Cu") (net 14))
 (segment (start 151.384 90.424) (end 152.146 89.662) (width 0.5334) (layer "B.Cu") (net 14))
 (segment (start 107.696 86.36) (end 106.934 87.122) (width 0.5334) (layer "B.Cu") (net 14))
 (segment (start 118.628 85.588) (end 117.856 86.36) (width 0.5334) (layer "B.Cu") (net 14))
 (segment (start 136.652 82.804) (end 144.272 90.424) (width 0.5334) (layer "B.Cu") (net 14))
 (segment (start 144.272 90.424) (end 151.384 90.424) (width 0.5334) (layer "B.Cu") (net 14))
 (segment (start 152.146 89.662) (end 152.146 87.376) (width 0.5334) (layer "B.Cu") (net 14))
 (segment (start 134.112 76.454) (end 118.648 76.454) (width 0.5334) (layer "B.Cu") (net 16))
 (segment (start 118.648 76.454) (end 118.628 76.474) (width 0.5334) (layer "B.Cu") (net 16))
 (segment (start 114.574 79.014) (end 115.824 80.264) (width 0.5334) (layer "B.Cu") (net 12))
 (segment (start 137.668 80.264) (end 146.558 89.154) (width 0.5334) (layer "B.Cu") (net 12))
 (segment (start 115.824 80.264) (end 137.668 80.264) (width 0.5334) (layer "B.Cu") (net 12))
 (segment (start 111.008 79.014) (end 114.574 79.014) (width 0.5334) (layer "B.Cu") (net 12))
 (segment (start 146.558 89.154) (end 149.352 89.154) (width 0.5334) (layer "B.Cu") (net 12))
 (segment (start 118.648 73.914) (end 118.628 73.934) (width 0.5334) (layer "B.Cu") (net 17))
 (segment (start 134.112 73.914) (end 118.648 73.914) (width 0.5334) (layer "B.Cu") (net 17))
 (segment (start 118.648 71.374) (end 118.628 71.394) (width 0.5334) (layer "B.Cu") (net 18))
 (segment (start 134.112 71.374) (end 118.648 71.374) (width 0.5334) (layer "B.Cu") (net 18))
 (segment (start 119.126 99.568) (end 110.236 99.568) (width 0.5334) (layer "B.Cu") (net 1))
 (segment (start 119.38 90.424) (end 109.982 90.424) (width 0.5334) (layer "B.Cu") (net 3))
 (segment (start 102.362 94.996) (end 102.326 94.96) (width 0.5334) (layer "B.Cu") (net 29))
 (segment (start 102.326 101.056) (end 102.326 94.96) (width 0.5334) (layer "B.Cu") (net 29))
 (segment (start 130.048 100.838) (end 128.836499 102.049501) (width 0.5334) (layer "B.Cu") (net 29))
 (segment (start 130.048 88.392) (end 130.048 100.838) (width 0.5334) (layer "B.Cu") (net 29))
 (segment (start 128.836499 102.049501) (end 103.319501 102.049501) (width 0.5334) (layer "B.Cu") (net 29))
 (segment (start 134.112 86.614) (end 131.826 86.614) (width 0.5334) (layer "B.Cu") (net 29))
 (segment (start 103.319501 102.049501) (end 102.326 101.056) (width 0.5334) (layer "B.Cu") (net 29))
 (segment (start 131.826 86.614) (end 130.048 88.392) (width 0.5334) (layer "B.Cu") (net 29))
 (segment (start 109.982 94.996) (end 102.362 94.996) (width 0.5334) (layer "B.Cu") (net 29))
 (segment (start 102.326 94.96) (end 102.326 79.248) (width 0.5334) (layer "B.Cu") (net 29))
 (segment (start 102.326 72.748) (end 102.326 79.248) (width 0.5334) (layer "B.Cu") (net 29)))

